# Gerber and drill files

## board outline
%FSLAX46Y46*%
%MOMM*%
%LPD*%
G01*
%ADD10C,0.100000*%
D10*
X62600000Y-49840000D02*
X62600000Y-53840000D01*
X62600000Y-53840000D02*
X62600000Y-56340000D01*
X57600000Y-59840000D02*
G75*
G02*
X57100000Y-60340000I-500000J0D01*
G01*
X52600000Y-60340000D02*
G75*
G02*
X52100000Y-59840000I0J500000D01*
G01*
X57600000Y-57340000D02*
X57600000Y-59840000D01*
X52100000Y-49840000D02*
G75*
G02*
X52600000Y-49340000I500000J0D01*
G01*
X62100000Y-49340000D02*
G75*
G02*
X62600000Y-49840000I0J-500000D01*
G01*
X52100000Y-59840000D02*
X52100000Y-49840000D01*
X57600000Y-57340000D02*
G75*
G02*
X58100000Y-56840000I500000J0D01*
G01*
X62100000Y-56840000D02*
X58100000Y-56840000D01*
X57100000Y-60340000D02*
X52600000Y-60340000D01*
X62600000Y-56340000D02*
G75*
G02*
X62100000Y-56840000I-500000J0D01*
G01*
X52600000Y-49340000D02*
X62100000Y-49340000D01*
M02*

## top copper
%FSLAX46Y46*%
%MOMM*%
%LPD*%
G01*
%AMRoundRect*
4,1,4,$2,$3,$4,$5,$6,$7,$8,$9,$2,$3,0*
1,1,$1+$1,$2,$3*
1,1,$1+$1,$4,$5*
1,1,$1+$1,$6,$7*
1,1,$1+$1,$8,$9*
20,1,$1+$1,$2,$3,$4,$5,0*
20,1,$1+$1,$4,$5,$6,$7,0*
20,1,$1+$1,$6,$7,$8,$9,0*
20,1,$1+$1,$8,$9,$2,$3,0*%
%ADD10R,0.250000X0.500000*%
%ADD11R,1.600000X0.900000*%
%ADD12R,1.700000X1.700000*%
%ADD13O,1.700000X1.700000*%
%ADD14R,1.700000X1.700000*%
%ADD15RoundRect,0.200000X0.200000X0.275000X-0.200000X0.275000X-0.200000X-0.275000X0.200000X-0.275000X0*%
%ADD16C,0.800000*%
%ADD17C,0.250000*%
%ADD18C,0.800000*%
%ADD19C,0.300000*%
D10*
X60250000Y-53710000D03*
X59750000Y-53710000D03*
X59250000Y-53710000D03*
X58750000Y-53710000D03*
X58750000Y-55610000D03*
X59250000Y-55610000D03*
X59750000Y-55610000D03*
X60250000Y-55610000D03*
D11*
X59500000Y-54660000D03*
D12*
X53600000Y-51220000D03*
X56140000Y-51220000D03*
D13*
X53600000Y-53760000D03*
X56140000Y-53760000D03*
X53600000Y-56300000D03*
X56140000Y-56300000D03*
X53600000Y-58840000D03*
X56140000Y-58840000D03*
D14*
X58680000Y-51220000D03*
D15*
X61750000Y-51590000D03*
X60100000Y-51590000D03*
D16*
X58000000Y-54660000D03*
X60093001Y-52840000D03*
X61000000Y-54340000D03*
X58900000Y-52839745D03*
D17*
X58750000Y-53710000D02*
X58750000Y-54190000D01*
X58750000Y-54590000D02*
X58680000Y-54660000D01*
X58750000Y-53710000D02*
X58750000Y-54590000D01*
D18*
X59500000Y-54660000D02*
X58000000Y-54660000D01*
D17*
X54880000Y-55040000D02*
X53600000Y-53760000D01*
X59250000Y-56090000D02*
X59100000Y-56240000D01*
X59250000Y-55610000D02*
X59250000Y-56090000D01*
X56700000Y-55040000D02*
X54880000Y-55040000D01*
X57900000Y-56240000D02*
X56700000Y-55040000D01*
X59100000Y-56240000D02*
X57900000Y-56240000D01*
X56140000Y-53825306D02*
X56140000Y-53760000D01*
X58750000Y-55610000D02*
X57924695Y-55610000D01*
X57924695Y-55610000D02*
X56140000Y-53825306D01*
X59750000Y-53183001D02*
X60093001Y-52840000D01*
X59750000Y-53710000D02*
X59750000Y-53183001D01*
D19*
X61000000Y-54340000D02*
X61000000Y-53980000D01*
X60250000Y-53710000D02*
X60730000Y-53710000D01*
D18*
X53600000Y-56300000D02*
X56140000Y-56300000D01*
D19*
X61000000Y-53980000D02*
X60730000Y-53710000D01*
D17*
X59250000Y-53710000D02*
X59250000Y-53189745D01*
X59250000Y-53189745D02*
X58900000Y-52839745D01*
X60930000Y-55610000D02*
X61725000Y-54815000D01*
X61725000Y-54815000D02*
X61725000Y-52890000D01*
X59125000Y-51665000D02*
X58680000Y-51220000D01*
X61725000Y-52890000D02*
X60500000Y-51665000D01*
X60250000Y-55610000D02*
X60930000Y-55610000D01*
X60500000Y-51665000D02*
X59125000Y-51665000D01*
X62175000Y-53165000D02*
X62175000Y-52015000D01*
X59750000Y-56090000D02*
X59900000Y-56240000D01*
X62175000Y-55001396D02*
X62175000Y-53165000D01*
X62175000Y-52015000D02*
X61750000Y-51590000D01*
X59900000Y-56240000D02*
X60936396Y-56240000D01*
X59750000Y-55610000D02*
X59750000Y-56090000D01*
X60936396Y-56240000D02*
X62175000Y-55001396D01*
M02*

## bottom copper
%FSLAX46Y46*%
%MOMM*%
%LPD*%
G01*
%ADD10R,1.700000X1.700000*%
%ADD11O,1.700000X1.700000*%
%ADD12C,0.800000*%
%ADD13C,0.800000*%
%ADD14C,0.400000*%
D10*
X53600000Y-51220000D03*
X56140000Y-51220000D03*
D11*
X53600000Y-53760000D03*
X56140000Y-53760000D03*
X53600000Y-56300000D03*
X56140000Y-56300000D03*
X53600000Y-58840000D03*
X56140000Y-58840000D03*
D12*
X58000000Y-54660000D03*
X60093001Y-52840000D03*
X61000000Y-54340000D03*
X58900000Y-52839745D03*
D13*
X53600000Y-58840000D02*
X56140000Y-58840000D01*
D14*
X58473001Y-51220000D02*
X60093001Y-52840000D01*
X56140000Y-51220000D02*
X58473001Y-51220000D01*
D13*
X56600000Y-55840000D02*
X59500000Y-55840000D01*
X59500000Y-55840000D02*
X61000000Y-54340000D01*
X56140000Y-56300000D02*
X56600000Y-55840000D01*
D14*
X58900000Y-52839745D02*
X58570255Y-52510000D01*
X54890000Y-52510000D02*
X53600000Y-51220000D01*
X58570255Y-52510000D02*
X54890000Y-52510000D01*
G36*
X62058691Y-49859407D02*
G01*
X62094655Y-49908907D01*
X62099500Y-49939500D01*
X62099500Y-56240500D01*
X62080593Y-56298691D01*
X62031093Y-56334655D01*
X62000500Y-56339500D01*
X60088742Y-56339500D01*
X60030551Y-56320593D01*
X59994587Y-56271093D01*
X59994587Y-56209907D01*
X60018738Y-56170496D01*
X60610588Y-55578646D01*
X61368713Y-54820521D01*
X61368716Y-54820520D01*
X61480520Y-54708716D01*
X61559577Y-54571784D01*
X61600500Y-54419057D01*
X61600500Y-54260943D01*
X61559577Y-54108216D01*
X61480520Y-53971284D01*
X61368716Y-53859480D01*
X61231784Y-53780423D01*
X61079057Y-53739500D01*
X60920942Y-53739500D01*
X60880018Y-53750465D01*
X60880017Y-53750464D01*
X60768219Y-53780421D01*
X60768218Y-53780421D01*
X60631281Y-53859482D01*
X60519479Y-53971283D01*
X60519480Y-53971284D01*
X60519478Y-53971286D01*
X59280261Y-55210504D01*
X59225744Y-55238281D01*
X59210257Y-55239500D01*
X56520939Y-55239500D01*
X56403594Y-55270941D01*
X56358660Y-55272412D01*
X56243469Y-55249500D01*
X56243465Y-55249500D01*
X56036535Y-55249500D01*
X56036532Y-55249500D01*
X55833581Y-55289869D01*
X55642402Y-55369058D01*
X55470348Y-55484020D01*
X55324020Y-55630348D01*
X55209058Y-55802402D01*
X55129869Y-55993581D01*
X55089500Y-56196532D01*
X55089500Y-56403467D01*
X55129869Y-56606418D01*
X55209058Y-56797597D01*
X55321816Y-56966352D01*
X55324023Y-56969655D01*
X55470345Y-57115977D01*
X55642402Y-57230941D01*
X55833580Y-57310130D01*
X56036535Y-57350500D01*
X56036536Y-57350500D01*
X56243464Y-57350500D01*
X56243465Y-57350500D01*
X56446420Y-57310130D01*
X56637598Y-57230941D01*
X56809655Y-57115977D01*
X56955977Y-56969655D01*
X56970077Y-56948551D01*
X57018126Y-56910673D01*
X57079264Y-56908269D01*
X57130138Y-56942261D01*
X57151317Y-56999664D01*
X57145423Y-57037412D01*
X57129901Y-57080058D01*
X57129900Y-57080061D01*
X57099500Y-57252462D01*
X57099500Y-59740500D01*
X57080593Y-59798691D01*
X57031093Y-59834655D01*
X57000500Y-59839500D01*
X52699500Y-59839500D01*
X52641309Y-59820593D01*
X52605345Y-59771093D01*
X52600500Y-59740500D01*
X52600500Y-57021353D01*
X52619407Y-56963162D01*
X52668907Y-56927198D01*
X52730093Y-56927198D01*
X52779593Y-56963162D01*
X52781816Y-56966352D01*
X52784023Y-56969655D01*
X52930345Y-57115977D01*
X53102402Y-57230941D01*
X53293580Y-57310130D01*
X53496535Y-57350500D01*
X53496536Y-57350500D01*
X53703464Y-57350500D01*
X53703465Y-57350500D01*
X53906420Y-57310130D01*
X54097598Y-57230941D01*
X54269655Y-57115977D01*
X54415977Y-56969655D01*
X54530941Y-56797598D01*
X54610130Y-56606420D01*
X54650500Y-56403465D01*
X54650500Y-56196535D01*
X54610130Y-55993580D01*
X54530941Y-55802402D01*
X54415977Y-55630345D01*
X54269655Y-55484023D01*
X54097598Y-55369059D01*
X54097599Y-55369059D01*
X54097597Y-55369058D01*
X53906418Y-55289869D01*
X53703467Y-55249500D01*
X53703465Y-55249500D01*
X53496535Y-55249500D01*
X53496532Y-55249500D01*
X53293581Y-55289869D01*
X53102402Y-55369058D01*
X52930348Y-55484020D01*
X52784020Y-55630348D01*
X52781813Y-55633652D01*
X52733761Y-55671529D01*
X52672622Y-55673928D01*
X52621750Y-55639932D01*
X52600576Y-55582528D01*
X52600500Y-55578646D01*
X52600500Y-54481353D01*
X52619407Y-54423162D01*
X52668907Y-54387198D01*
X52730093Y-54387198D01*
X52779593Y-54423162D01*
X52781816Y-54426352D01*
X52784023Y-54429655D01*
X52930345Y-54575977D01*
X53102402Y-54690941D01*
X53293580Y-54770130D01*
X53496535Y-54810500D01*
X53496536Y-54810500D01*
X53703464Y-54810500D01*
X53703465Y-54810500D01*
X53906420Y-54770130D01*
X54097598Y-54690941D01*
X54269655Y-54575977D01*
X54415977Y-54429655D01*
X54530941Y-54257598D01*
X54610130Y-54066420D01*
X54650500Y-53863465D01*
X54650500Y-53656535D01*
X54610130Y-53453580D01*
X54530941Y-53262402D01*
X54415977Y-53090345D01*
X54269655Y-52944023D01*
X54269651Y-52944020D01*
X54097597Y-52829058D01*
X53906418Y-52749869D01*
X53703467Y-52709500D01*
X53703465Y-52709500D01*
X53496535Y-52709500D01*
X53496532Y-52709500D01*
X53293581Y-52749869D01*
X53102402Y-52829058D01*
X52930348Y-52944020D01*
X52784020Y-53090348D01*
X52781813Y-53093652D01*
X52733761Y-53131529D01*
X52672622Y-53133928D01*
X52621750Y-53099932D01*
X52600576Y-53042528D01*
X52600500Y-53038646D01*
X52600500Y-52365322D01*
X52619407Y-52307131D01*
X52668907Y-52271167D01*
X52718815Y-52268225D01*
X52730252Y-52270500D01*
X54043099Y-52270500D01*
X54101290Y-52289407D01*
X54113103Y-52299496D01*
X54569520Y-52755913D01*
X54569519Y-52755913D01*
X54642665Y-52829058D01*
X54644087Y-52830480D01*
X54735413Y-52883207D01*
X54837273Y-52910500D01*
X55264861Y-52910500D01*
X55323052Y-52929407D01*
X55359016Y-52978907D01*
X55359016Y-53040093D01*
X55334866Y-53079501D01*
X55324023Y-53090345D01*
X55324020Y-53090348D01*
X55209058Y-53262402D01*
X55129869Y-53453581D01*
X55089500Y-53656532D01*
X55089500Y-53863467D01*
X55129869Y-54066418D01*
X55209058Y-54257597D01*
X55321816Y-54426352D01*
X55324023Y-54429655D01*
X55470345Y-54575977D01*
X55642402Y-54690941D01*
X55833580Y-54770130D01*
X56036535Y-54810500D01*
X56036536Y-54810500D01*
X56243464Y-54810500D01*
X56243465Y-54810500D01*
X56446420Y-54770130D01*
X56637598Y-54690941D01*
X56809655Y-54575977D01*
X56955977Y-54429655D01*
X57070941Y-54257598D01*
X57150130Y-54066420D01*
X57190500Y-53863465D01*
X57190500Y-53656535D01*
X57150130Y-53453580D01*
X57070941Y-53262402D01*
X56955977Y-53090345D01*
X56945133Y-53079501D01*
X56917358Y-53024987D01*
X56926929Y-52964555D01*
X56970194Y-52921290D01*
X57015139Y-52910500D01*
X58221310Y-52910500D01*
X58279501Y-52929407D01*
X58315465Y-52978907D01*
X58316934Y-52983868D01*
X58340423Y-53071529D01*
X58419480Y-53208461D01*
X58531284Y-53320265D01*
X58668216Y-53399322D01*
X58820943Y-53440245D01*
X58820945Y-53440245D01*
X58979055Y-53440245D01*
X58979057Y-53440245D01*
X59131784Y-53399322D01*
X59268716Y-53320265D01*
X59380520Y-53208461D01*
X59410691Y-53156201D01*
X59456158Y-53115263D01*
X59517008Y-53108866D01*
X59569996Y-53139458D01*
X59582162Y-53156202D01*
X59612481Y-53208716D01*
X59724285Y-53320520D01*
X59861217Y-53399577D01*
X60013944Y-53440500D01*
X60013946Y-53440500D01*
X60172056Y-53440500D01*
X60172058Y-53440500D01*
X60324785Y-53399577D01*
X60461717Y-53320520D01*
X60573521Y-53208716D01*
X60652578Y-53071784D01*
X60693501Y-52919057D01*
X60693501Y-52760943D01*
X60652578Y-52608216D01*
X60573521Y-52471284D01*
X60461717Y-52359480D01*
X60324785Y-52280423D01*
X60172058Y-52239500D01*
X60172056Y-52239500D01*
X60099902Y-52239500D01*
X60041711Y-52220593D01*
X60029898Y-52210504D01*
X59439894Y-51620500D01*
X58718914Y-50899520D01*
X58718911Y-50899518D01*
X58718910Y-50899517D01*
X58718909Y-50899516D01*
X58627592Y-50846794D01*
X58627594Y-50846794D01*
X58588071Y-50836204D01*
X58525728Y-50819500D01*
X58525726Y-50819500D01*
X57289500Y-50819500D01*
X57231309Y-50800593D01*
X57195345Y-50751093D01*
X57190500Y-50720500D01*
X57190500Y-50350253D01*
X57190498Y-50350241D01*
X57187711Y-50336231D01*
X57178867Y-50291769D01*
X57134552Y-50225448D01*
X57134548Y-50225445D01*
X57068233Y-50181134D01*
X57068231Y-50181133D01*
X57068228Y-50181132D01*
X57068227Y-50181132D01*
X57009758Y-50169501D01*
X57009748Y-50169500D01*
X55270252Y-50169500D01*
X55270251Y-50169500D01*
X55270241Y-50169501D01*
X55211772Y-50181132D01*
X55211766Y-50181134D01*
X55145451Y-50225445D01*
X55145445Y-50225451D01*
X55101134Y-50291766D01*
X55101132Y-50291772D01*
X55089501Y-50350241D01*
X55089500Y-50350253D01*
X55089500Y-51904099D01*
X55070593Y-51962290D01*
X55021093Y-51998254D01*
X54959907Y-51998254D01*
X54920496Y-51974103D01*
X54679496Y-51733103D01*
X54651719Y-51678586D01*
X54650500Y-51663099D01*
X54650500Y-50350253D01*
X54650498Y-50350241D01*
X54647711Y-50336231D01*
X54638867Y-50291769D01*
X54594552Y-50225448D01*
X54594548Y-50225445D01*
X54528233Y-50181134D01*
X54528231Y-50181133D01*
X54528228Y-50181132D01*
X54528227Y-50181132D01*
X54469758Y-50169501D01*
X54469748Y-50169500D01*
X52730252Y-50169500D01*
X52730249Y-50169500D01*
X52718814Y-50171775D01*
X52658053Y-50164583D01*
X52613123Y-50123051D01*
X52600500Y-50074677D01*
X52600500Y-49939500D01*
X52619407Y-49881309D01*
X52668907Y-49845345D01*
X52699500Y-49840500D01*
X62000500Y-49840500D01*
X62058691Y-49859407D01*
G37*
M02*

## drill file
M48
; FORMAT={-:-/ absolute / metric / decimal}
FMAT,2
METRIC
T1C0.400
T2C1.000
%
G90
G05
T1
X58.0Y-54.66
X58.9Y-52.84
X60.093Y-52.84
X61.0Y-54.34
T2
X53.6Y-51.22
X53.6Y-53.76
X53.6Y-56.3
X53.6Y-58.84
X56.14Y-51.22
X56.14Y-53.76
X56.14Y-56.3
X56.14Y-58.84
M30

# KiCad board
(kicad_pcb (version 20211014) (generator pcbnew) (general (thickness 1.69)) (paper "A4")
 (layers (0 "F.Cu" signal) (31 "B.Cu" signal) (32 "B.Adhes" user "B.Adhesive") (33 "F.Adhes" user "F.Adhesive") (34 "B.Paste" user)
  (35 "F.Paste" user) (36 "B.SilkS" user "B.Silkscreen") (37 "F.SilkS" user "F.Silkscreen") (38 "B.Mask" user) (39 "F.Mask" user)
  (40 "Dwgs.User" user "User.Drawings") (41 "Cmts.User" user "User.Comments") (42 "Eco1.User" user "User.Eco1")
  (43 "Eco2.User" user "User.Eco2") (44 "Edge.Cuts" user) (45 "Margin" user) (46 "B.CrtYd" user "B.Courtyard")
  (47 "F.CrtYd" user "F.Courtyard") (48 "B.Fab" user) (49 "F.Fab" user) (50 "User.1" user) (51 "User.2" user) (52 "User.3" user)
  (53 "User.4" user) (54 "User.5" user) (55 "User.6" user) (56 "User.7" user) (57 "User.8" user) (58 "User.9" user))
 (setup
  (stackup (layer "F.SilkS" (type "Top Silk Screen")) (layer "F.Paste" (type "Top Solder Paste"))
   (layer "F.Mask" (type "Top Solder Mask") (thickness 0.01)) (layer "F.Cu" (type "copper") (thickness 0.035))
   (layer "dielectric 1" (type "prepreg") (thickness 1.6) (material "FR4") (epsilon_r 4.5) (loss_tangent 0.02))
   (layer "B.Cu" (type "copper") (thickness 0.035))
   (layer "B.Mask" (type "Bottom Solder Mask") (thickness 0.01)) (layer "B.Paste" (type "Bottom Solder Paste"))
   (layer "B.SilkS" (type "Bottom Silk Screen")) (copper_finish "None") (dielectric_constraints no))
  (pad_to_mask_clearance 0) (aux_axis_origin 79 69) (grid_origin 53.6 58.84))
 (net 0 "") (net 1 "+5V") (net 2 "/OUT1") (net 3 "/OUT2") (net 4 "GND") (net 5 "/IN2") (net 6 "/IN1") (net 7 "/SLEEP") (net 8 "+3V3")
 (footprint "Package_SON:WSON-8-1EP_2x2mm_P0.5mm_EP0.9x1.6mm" (layer "F.Cu") (at 59.5 54.66 -90)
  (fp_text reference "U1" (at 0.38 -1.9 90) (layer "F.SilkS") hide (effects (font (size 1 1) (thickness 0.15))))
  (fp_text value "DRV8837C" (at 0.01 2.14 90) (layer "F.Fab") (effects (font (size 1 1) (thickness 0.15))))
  (pad "" smd rect (at 0 -0.4 270) (size 0.75 0.65) (layers "F.Paste"))
  (pad "" smd rect (at 0 0.4 270) (size 0.75 0.65) (layers "F.Paste"))
  (pad "1" smd rect (at -0.95 -0.75 270) (size 0.5 0.25) (layers "F.Cu" "F.Paste" "F.Mask") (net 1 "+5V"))
  (pad "2" smd rect (at -0.95 -0.25 270) (size 0.5 0.25) (layers "F.Cu" "F.Paste" "F.Mask") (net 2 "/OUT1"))
  (pad "3" smd rect (at -0.95 0.25 270) (size 0.5 0.25) (layers "F.Cu" "F.Paste" "F.Mask") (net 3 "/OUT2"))
  (pad "4" smd rect (at -0.95 0.75 270) (size 0.5 0.25) (layers "F.Cu" "F.Paste" "F.Mask") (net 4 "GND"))
  (pad "5" smd rect (at 0.95 0.75 270) (size 0.5 0.25) (layers "F.Cu" "F.Paste" "F.Mask") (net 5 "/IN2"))
  (pad "6" smd rect (at 0.95 0.25 270) (size 0.5 0.25) (layers "F.Cu" "F.Paste" "F.Mask") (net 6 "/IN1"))
  (pad "7" smd rect (at 0.95 -0.25 270) (size 0.5 0.25) (layers "F.Cu" "F.Paste" "F.Mask") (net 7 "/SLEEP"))
  (pad "8" smd rect (at 0.95 -0.75 270) (size 0.5 0.25) (layers "F.Cu" "F.Paste" "F.Mask") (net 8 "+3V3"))
  (pad "9" smd rect (at 0 0 270) (size 0.9 1.6) (layers "F.Cu" "F.Mask") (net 4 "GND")))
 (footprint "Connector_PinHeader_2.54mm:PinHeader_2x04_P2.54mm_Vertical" (layer "F.Cu") (at 53.6 51.22)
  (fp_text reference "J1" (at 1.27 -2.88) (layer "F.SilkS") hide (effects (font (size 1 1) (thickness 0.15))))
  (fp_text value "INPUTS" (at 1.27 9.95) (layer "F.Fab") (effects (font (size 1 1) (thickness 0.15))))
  (pad "1" thru_hole rect (at 0 0) (size 1.7 1.7) (drill 1) (layers *.Cu *.Mask) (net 3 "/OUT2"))
  (pad "2" thru_hole rect (at 2.54 0) (size 1.7 1.7) (drill 1) (layers *.Cu *.Mask) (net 2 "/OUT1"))
  (pad "3" thru_hole oval (at 0 2.54) (size 1.7 1.7) (drill 1) (layers *.Cu *.Mask) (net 6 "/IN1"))
  (pad "4" thru_hole oval (at 2.54 2.54) (size 1.7 1.7) (drill 1) (layers *.Cu *.Mask) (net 5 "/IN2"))
  (pad "5" thru_hole oval (at 0 5.08) (size 1.7 1.7) (drill 1) (layers *.Cu *.Mask) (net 1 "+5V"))
  (pad "6" thru_hole oval (at 2.54 5.08) (size 1.7 1.7) (drill 1) (layers *.Cu *.Mask) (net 1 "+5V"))
  (pad "7" thru_hole oval (at 0 7.62) (size 1.7 1.7) (drill 1) (layers *.Cu *.Mask) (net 4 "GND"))
  (pad "8" thru_hole oval (at 2.54 7.62) (size 1.7 1.7) (drill 1) (layers *.Cu *.Mask) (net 4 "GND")))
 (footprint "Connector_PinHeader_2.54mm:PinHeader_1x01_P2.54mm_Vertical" (layer "F.Cu") (at 58.68 51.22)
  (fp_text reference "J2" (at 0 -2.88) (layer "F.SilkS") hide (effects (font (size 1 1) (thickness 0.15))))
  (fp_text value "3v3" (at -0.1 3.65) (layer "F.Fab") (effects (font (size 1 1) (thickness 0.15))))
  (pad "1" smd rect (at 0 0) (size 1.7 1.7) (layers "F.Cu" "F.Paste" "F.Mask") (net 8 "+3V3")))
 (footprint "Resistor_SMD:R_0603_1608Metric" (layer "F.Cu") (at 60.925 51.59 180)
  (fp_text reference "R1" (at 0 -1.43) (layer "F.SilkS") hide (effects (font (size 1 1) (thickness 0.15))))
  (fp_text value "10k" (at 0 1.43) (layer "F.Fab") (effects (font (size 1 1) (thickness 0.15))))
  (pad "1" smd roundrect (at -0.825 0 180) (size 0.8 0.95) (layers "F.Cu" "F.Paste" "F.Mask") (roundrect_rratio 0.25) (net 7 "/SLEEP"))
  (pad "2" smd roundrect (at 0.825 0 180) (size 0.8 0.95) (layers "F.Cu" "F.Paste" "F.Mask") (roundrect_rratio 0.25) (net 8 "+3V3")))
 (gr_line (start 62.6 49.84) (end 62.6 53.84) (layer "Edge.Cuts") (width 0.1))
 (gr_line (start 62.6 53.84) (end 62.6 56.34) (layer "Edge.Cuts") (width 0.1))
 (gr_arc (start 57.6 59.84) (mid 57.453553 60.193553) (end 57.1 60.34) (layer "Edge.Cuts") (width 0.1))
 (gr_arc (start 52.6 60.34) (mid 52.246447 60.193553) (end 52.1 59.84) (layer "Edge.Cuts") (width 0.1))
 (gr_line (start 57.6 57.34) (end 57.6 59.84) (layer "Edge.Cuts") (width 0.1))
 (gr_arc (start 52.1 49.84) (mid 52.246447 49.486447) (end 52.6 49.34) (layer "Edge.Cuts") (width 0.1))
 (gr_arc (start 62.1 49.34) (mid 62.453553 49.486447) (end 62.6 49.84) (layer "Edge.Cuts") (width 0.1))
 (gr_line (start 52.1 59.84) (end 52.1 49.84) (layer "Edge.Cuts") (width 0.1))
 (gr_arc (start 57.6 57.34) (mid 57.746447 56.986447) (end 58.1 56.84) (layer "Edge.Cuts") (width 0.1))
 (gr_line (start 62.1 56.84) (end 58.1 56.84) (layer "Edge.Cuts") (width 0.1))
 (gr_line (start 57.1 60.34) (end 52.6 60.34) (layer "Edge.Cuts") (width 0.1))
 (gr_arc (start 62.6 56.34) (mid 62.453553 56.693553) (end 62.1 56.84) (layer "Edge.Cuts") (width 0.1))
 (gr_line (start 52.6 49.34) (end 62.1 49.34) (layer "Edge.Cuts") (width 0.1))
 (segment (start 58.75 53.71) (end 58.75 54.19) (width 0.25) (layer "F.Cu") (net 4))
 (segment (start 58.75 54.59) (end 58.68 54.66) (width 0.25) (layer "F.Cu") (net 4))
 (segment (start 58.75 53.71) (end 58.75 54.59) (width 0.25) (layer "F.Cu") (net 4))
 (segment (start 59.5 54.66) (end 58 54.66) (width 0.8) (layer "F.Cu") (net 4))
 (via (at 58 54.66) (size 0.8) (drill 0.4) (layers "F.Cu" "B.Cu") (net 4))
 (segment (start 53.6 58.84) (end 56.14 58.84) (width 0.8) (layer "B.Cu") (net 4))
 (segment (start 54.88 55.04) (end 53.6 53.76) (width 0.25) (layer "F.Cu") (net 6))
 (segment (start 59.25 56.09) (end 59.1 56.24) (width 0.25) (layer "F.Cu") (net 6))
 (segment (start 59.25 55.61) (end 59.25 56.09) (width 0.25) (layer "F.Cu") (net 6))
 (segment (start 56.7 55.04) (end 54.88 55.04) (width 0.25) (layer "F.Cu") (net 6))
 (segment (start 57.9 56.24) (end 56.7 55.04) (width 0.25) (layer "F.Cu") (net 6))
 (segment (start 59.1 56.24) (end 57.9 56.24) (width 0.25) (layer "F.Cu") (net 6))
 (segment (start 56.14 53.825306) (end 56.14 53.76) (width 0.25) (layer "F.Cu") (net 5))
 (segment (start 58.75 55.61) (end 57.924695 55.61) (width 0.25) (layer "F.Cu") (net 5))
 (segment (start 57.924695 55.61) (end 56.14 53.825306) (width 0.25) (layer "F.Cu") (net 5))
 (segment (start 59.75 53.183001) (end 60.093001 52.84) (width 0.25) (layer "F.Cu") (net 2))
 (segment (start 59.75 53.71) (end 59.75 53.183001) (width 0.25) (layer "F.Cu") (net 2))
 (via (at 60.093001 52.84) (size 0.8) (drill 0.4) (layers "F.Cu" "B.Cu") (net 2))
 (segment (start 58.473001 51.22) (end 60.093001 52.84) (width 0.4) (layer "B.Cu") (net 2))
 (segment (start 56.14 51.22) (end 58.473001 51.22) (width 0.4) (layer "B.Cu") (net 2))
 (segment (start 61 54.34) (end 61 53.98) (width 0.3) (layer "F.Cu") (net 1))
 (segment (start 60.25 53.71) (end 60.73 53.71) (width 0.3) (layer "F.Cu") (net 1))
 (segment (start 53.6 56.3) (end 56.14 56.3) (width 0.8) (layer "F.Cu") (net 1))
 (segment (start 61 53.98) (end 60.73 53.71) (width 0.3) (layer "F.Cu") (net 1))
 (via (at 61 54.34) (size 0.8) (drill 0.4) (layers "F.Cu" "B.Cu") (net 1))
 (segment (start 56.6 55.84) (end 59.5 55.84) (width 0.8) (layer "B.Cu") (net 1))
 (segment (start 59.5 55.84) (end 61 54.34) (width 0.8) (layer "B.Cu") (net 1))
 (segment (start 56.14 56.3) (end 56.6 55.84) (width 0.8) (layer "B.Cu") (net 1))
 (segment (start 59.25 53.71) (end 59.25 53.189745) (width 0.25) (layer "F.Cu") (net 3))
 (segment (start 59.25 53.189745) (end 58.9 52.839745) (width 0.25) (layer "F.Cu") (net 3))
 (via (at 58.9 52.839745) (size 0.8) (drill 0.4) (layers "F.Cu" "B.Cu") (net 3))
 (segment (start 58.9 52.839745) (end 58.570255 52.51) (width 0.4) (layer "B.Cu") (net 3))
 (segment (start 54.89 52.51) (end 53.6 51.22) (width 0.4) (layer "B.Cu") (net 3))
 (segment (start 58.570255 52.51) (end 54.89 52.51) (width 0.4) (layer "B.Cu") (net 3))
 (segment (start 60.93 55.61) (end 61.725 54.815) (width 0.25) (layer "F.Cu") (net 8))
 (segment (start 61.725 54.815) (end 61.725 52.89) (width 0.25) (layer "F.Cu") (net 8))
 (segment (start 59.125 51.665) (end 58.68 51.22) (width 0.25) (layer "F.Cu") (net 8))
 (segment (start 61.725 52.89) (end 60.5 51.665) (width 0.25) (layer "F.Cu") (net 8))
 (segment (start 60.25 55.61) (end 60.93 55.61) (width 0.25) (layer "F.Cu") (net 8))
 (segment (start 60.5 51.665) (end 59.125 51.665) (width 0.25) (layer "F.Cu") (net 8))
 (segment (start 62.175 53.165) (end 62.175 52.015) (width 0.25) (layer "F.Cu") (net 7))
 (segment (start 59.75 56.09) (end 59.9 56.24) (width 0.25) (layer "F.Cu") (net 7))
 (segment (start 62.175 55.001396) (end 62.175 53.165) (width 0.25) (layer "F.Cu") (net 7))
 (segment (start 62.175 52.015) (end 61.75 51.59) (width 0.25) (layer "F.Cu") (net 7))
 (segment (start 59.9 56.24) (end 60.936396 56.24) (width 0.25) (layer "F.Cu") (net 7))
 (segment (start 59.75 55.61) (end 59.75 56.09) (width 0.25) (layer "F.Cu") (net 7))
 (segment (start 60.936396 56.24) (end 62.175 55.001396) (width 0.25) (layer "F.Cu") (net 7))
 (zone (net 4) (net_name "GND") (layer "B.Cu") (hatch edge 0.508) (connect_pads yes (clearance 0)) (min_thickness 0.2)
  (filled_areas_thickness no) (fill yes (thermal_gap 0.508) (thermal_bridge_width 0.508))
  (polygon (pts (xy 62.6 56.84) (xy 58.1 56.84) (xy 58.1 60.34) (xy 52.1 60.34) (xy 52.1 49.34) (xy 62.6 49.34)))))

